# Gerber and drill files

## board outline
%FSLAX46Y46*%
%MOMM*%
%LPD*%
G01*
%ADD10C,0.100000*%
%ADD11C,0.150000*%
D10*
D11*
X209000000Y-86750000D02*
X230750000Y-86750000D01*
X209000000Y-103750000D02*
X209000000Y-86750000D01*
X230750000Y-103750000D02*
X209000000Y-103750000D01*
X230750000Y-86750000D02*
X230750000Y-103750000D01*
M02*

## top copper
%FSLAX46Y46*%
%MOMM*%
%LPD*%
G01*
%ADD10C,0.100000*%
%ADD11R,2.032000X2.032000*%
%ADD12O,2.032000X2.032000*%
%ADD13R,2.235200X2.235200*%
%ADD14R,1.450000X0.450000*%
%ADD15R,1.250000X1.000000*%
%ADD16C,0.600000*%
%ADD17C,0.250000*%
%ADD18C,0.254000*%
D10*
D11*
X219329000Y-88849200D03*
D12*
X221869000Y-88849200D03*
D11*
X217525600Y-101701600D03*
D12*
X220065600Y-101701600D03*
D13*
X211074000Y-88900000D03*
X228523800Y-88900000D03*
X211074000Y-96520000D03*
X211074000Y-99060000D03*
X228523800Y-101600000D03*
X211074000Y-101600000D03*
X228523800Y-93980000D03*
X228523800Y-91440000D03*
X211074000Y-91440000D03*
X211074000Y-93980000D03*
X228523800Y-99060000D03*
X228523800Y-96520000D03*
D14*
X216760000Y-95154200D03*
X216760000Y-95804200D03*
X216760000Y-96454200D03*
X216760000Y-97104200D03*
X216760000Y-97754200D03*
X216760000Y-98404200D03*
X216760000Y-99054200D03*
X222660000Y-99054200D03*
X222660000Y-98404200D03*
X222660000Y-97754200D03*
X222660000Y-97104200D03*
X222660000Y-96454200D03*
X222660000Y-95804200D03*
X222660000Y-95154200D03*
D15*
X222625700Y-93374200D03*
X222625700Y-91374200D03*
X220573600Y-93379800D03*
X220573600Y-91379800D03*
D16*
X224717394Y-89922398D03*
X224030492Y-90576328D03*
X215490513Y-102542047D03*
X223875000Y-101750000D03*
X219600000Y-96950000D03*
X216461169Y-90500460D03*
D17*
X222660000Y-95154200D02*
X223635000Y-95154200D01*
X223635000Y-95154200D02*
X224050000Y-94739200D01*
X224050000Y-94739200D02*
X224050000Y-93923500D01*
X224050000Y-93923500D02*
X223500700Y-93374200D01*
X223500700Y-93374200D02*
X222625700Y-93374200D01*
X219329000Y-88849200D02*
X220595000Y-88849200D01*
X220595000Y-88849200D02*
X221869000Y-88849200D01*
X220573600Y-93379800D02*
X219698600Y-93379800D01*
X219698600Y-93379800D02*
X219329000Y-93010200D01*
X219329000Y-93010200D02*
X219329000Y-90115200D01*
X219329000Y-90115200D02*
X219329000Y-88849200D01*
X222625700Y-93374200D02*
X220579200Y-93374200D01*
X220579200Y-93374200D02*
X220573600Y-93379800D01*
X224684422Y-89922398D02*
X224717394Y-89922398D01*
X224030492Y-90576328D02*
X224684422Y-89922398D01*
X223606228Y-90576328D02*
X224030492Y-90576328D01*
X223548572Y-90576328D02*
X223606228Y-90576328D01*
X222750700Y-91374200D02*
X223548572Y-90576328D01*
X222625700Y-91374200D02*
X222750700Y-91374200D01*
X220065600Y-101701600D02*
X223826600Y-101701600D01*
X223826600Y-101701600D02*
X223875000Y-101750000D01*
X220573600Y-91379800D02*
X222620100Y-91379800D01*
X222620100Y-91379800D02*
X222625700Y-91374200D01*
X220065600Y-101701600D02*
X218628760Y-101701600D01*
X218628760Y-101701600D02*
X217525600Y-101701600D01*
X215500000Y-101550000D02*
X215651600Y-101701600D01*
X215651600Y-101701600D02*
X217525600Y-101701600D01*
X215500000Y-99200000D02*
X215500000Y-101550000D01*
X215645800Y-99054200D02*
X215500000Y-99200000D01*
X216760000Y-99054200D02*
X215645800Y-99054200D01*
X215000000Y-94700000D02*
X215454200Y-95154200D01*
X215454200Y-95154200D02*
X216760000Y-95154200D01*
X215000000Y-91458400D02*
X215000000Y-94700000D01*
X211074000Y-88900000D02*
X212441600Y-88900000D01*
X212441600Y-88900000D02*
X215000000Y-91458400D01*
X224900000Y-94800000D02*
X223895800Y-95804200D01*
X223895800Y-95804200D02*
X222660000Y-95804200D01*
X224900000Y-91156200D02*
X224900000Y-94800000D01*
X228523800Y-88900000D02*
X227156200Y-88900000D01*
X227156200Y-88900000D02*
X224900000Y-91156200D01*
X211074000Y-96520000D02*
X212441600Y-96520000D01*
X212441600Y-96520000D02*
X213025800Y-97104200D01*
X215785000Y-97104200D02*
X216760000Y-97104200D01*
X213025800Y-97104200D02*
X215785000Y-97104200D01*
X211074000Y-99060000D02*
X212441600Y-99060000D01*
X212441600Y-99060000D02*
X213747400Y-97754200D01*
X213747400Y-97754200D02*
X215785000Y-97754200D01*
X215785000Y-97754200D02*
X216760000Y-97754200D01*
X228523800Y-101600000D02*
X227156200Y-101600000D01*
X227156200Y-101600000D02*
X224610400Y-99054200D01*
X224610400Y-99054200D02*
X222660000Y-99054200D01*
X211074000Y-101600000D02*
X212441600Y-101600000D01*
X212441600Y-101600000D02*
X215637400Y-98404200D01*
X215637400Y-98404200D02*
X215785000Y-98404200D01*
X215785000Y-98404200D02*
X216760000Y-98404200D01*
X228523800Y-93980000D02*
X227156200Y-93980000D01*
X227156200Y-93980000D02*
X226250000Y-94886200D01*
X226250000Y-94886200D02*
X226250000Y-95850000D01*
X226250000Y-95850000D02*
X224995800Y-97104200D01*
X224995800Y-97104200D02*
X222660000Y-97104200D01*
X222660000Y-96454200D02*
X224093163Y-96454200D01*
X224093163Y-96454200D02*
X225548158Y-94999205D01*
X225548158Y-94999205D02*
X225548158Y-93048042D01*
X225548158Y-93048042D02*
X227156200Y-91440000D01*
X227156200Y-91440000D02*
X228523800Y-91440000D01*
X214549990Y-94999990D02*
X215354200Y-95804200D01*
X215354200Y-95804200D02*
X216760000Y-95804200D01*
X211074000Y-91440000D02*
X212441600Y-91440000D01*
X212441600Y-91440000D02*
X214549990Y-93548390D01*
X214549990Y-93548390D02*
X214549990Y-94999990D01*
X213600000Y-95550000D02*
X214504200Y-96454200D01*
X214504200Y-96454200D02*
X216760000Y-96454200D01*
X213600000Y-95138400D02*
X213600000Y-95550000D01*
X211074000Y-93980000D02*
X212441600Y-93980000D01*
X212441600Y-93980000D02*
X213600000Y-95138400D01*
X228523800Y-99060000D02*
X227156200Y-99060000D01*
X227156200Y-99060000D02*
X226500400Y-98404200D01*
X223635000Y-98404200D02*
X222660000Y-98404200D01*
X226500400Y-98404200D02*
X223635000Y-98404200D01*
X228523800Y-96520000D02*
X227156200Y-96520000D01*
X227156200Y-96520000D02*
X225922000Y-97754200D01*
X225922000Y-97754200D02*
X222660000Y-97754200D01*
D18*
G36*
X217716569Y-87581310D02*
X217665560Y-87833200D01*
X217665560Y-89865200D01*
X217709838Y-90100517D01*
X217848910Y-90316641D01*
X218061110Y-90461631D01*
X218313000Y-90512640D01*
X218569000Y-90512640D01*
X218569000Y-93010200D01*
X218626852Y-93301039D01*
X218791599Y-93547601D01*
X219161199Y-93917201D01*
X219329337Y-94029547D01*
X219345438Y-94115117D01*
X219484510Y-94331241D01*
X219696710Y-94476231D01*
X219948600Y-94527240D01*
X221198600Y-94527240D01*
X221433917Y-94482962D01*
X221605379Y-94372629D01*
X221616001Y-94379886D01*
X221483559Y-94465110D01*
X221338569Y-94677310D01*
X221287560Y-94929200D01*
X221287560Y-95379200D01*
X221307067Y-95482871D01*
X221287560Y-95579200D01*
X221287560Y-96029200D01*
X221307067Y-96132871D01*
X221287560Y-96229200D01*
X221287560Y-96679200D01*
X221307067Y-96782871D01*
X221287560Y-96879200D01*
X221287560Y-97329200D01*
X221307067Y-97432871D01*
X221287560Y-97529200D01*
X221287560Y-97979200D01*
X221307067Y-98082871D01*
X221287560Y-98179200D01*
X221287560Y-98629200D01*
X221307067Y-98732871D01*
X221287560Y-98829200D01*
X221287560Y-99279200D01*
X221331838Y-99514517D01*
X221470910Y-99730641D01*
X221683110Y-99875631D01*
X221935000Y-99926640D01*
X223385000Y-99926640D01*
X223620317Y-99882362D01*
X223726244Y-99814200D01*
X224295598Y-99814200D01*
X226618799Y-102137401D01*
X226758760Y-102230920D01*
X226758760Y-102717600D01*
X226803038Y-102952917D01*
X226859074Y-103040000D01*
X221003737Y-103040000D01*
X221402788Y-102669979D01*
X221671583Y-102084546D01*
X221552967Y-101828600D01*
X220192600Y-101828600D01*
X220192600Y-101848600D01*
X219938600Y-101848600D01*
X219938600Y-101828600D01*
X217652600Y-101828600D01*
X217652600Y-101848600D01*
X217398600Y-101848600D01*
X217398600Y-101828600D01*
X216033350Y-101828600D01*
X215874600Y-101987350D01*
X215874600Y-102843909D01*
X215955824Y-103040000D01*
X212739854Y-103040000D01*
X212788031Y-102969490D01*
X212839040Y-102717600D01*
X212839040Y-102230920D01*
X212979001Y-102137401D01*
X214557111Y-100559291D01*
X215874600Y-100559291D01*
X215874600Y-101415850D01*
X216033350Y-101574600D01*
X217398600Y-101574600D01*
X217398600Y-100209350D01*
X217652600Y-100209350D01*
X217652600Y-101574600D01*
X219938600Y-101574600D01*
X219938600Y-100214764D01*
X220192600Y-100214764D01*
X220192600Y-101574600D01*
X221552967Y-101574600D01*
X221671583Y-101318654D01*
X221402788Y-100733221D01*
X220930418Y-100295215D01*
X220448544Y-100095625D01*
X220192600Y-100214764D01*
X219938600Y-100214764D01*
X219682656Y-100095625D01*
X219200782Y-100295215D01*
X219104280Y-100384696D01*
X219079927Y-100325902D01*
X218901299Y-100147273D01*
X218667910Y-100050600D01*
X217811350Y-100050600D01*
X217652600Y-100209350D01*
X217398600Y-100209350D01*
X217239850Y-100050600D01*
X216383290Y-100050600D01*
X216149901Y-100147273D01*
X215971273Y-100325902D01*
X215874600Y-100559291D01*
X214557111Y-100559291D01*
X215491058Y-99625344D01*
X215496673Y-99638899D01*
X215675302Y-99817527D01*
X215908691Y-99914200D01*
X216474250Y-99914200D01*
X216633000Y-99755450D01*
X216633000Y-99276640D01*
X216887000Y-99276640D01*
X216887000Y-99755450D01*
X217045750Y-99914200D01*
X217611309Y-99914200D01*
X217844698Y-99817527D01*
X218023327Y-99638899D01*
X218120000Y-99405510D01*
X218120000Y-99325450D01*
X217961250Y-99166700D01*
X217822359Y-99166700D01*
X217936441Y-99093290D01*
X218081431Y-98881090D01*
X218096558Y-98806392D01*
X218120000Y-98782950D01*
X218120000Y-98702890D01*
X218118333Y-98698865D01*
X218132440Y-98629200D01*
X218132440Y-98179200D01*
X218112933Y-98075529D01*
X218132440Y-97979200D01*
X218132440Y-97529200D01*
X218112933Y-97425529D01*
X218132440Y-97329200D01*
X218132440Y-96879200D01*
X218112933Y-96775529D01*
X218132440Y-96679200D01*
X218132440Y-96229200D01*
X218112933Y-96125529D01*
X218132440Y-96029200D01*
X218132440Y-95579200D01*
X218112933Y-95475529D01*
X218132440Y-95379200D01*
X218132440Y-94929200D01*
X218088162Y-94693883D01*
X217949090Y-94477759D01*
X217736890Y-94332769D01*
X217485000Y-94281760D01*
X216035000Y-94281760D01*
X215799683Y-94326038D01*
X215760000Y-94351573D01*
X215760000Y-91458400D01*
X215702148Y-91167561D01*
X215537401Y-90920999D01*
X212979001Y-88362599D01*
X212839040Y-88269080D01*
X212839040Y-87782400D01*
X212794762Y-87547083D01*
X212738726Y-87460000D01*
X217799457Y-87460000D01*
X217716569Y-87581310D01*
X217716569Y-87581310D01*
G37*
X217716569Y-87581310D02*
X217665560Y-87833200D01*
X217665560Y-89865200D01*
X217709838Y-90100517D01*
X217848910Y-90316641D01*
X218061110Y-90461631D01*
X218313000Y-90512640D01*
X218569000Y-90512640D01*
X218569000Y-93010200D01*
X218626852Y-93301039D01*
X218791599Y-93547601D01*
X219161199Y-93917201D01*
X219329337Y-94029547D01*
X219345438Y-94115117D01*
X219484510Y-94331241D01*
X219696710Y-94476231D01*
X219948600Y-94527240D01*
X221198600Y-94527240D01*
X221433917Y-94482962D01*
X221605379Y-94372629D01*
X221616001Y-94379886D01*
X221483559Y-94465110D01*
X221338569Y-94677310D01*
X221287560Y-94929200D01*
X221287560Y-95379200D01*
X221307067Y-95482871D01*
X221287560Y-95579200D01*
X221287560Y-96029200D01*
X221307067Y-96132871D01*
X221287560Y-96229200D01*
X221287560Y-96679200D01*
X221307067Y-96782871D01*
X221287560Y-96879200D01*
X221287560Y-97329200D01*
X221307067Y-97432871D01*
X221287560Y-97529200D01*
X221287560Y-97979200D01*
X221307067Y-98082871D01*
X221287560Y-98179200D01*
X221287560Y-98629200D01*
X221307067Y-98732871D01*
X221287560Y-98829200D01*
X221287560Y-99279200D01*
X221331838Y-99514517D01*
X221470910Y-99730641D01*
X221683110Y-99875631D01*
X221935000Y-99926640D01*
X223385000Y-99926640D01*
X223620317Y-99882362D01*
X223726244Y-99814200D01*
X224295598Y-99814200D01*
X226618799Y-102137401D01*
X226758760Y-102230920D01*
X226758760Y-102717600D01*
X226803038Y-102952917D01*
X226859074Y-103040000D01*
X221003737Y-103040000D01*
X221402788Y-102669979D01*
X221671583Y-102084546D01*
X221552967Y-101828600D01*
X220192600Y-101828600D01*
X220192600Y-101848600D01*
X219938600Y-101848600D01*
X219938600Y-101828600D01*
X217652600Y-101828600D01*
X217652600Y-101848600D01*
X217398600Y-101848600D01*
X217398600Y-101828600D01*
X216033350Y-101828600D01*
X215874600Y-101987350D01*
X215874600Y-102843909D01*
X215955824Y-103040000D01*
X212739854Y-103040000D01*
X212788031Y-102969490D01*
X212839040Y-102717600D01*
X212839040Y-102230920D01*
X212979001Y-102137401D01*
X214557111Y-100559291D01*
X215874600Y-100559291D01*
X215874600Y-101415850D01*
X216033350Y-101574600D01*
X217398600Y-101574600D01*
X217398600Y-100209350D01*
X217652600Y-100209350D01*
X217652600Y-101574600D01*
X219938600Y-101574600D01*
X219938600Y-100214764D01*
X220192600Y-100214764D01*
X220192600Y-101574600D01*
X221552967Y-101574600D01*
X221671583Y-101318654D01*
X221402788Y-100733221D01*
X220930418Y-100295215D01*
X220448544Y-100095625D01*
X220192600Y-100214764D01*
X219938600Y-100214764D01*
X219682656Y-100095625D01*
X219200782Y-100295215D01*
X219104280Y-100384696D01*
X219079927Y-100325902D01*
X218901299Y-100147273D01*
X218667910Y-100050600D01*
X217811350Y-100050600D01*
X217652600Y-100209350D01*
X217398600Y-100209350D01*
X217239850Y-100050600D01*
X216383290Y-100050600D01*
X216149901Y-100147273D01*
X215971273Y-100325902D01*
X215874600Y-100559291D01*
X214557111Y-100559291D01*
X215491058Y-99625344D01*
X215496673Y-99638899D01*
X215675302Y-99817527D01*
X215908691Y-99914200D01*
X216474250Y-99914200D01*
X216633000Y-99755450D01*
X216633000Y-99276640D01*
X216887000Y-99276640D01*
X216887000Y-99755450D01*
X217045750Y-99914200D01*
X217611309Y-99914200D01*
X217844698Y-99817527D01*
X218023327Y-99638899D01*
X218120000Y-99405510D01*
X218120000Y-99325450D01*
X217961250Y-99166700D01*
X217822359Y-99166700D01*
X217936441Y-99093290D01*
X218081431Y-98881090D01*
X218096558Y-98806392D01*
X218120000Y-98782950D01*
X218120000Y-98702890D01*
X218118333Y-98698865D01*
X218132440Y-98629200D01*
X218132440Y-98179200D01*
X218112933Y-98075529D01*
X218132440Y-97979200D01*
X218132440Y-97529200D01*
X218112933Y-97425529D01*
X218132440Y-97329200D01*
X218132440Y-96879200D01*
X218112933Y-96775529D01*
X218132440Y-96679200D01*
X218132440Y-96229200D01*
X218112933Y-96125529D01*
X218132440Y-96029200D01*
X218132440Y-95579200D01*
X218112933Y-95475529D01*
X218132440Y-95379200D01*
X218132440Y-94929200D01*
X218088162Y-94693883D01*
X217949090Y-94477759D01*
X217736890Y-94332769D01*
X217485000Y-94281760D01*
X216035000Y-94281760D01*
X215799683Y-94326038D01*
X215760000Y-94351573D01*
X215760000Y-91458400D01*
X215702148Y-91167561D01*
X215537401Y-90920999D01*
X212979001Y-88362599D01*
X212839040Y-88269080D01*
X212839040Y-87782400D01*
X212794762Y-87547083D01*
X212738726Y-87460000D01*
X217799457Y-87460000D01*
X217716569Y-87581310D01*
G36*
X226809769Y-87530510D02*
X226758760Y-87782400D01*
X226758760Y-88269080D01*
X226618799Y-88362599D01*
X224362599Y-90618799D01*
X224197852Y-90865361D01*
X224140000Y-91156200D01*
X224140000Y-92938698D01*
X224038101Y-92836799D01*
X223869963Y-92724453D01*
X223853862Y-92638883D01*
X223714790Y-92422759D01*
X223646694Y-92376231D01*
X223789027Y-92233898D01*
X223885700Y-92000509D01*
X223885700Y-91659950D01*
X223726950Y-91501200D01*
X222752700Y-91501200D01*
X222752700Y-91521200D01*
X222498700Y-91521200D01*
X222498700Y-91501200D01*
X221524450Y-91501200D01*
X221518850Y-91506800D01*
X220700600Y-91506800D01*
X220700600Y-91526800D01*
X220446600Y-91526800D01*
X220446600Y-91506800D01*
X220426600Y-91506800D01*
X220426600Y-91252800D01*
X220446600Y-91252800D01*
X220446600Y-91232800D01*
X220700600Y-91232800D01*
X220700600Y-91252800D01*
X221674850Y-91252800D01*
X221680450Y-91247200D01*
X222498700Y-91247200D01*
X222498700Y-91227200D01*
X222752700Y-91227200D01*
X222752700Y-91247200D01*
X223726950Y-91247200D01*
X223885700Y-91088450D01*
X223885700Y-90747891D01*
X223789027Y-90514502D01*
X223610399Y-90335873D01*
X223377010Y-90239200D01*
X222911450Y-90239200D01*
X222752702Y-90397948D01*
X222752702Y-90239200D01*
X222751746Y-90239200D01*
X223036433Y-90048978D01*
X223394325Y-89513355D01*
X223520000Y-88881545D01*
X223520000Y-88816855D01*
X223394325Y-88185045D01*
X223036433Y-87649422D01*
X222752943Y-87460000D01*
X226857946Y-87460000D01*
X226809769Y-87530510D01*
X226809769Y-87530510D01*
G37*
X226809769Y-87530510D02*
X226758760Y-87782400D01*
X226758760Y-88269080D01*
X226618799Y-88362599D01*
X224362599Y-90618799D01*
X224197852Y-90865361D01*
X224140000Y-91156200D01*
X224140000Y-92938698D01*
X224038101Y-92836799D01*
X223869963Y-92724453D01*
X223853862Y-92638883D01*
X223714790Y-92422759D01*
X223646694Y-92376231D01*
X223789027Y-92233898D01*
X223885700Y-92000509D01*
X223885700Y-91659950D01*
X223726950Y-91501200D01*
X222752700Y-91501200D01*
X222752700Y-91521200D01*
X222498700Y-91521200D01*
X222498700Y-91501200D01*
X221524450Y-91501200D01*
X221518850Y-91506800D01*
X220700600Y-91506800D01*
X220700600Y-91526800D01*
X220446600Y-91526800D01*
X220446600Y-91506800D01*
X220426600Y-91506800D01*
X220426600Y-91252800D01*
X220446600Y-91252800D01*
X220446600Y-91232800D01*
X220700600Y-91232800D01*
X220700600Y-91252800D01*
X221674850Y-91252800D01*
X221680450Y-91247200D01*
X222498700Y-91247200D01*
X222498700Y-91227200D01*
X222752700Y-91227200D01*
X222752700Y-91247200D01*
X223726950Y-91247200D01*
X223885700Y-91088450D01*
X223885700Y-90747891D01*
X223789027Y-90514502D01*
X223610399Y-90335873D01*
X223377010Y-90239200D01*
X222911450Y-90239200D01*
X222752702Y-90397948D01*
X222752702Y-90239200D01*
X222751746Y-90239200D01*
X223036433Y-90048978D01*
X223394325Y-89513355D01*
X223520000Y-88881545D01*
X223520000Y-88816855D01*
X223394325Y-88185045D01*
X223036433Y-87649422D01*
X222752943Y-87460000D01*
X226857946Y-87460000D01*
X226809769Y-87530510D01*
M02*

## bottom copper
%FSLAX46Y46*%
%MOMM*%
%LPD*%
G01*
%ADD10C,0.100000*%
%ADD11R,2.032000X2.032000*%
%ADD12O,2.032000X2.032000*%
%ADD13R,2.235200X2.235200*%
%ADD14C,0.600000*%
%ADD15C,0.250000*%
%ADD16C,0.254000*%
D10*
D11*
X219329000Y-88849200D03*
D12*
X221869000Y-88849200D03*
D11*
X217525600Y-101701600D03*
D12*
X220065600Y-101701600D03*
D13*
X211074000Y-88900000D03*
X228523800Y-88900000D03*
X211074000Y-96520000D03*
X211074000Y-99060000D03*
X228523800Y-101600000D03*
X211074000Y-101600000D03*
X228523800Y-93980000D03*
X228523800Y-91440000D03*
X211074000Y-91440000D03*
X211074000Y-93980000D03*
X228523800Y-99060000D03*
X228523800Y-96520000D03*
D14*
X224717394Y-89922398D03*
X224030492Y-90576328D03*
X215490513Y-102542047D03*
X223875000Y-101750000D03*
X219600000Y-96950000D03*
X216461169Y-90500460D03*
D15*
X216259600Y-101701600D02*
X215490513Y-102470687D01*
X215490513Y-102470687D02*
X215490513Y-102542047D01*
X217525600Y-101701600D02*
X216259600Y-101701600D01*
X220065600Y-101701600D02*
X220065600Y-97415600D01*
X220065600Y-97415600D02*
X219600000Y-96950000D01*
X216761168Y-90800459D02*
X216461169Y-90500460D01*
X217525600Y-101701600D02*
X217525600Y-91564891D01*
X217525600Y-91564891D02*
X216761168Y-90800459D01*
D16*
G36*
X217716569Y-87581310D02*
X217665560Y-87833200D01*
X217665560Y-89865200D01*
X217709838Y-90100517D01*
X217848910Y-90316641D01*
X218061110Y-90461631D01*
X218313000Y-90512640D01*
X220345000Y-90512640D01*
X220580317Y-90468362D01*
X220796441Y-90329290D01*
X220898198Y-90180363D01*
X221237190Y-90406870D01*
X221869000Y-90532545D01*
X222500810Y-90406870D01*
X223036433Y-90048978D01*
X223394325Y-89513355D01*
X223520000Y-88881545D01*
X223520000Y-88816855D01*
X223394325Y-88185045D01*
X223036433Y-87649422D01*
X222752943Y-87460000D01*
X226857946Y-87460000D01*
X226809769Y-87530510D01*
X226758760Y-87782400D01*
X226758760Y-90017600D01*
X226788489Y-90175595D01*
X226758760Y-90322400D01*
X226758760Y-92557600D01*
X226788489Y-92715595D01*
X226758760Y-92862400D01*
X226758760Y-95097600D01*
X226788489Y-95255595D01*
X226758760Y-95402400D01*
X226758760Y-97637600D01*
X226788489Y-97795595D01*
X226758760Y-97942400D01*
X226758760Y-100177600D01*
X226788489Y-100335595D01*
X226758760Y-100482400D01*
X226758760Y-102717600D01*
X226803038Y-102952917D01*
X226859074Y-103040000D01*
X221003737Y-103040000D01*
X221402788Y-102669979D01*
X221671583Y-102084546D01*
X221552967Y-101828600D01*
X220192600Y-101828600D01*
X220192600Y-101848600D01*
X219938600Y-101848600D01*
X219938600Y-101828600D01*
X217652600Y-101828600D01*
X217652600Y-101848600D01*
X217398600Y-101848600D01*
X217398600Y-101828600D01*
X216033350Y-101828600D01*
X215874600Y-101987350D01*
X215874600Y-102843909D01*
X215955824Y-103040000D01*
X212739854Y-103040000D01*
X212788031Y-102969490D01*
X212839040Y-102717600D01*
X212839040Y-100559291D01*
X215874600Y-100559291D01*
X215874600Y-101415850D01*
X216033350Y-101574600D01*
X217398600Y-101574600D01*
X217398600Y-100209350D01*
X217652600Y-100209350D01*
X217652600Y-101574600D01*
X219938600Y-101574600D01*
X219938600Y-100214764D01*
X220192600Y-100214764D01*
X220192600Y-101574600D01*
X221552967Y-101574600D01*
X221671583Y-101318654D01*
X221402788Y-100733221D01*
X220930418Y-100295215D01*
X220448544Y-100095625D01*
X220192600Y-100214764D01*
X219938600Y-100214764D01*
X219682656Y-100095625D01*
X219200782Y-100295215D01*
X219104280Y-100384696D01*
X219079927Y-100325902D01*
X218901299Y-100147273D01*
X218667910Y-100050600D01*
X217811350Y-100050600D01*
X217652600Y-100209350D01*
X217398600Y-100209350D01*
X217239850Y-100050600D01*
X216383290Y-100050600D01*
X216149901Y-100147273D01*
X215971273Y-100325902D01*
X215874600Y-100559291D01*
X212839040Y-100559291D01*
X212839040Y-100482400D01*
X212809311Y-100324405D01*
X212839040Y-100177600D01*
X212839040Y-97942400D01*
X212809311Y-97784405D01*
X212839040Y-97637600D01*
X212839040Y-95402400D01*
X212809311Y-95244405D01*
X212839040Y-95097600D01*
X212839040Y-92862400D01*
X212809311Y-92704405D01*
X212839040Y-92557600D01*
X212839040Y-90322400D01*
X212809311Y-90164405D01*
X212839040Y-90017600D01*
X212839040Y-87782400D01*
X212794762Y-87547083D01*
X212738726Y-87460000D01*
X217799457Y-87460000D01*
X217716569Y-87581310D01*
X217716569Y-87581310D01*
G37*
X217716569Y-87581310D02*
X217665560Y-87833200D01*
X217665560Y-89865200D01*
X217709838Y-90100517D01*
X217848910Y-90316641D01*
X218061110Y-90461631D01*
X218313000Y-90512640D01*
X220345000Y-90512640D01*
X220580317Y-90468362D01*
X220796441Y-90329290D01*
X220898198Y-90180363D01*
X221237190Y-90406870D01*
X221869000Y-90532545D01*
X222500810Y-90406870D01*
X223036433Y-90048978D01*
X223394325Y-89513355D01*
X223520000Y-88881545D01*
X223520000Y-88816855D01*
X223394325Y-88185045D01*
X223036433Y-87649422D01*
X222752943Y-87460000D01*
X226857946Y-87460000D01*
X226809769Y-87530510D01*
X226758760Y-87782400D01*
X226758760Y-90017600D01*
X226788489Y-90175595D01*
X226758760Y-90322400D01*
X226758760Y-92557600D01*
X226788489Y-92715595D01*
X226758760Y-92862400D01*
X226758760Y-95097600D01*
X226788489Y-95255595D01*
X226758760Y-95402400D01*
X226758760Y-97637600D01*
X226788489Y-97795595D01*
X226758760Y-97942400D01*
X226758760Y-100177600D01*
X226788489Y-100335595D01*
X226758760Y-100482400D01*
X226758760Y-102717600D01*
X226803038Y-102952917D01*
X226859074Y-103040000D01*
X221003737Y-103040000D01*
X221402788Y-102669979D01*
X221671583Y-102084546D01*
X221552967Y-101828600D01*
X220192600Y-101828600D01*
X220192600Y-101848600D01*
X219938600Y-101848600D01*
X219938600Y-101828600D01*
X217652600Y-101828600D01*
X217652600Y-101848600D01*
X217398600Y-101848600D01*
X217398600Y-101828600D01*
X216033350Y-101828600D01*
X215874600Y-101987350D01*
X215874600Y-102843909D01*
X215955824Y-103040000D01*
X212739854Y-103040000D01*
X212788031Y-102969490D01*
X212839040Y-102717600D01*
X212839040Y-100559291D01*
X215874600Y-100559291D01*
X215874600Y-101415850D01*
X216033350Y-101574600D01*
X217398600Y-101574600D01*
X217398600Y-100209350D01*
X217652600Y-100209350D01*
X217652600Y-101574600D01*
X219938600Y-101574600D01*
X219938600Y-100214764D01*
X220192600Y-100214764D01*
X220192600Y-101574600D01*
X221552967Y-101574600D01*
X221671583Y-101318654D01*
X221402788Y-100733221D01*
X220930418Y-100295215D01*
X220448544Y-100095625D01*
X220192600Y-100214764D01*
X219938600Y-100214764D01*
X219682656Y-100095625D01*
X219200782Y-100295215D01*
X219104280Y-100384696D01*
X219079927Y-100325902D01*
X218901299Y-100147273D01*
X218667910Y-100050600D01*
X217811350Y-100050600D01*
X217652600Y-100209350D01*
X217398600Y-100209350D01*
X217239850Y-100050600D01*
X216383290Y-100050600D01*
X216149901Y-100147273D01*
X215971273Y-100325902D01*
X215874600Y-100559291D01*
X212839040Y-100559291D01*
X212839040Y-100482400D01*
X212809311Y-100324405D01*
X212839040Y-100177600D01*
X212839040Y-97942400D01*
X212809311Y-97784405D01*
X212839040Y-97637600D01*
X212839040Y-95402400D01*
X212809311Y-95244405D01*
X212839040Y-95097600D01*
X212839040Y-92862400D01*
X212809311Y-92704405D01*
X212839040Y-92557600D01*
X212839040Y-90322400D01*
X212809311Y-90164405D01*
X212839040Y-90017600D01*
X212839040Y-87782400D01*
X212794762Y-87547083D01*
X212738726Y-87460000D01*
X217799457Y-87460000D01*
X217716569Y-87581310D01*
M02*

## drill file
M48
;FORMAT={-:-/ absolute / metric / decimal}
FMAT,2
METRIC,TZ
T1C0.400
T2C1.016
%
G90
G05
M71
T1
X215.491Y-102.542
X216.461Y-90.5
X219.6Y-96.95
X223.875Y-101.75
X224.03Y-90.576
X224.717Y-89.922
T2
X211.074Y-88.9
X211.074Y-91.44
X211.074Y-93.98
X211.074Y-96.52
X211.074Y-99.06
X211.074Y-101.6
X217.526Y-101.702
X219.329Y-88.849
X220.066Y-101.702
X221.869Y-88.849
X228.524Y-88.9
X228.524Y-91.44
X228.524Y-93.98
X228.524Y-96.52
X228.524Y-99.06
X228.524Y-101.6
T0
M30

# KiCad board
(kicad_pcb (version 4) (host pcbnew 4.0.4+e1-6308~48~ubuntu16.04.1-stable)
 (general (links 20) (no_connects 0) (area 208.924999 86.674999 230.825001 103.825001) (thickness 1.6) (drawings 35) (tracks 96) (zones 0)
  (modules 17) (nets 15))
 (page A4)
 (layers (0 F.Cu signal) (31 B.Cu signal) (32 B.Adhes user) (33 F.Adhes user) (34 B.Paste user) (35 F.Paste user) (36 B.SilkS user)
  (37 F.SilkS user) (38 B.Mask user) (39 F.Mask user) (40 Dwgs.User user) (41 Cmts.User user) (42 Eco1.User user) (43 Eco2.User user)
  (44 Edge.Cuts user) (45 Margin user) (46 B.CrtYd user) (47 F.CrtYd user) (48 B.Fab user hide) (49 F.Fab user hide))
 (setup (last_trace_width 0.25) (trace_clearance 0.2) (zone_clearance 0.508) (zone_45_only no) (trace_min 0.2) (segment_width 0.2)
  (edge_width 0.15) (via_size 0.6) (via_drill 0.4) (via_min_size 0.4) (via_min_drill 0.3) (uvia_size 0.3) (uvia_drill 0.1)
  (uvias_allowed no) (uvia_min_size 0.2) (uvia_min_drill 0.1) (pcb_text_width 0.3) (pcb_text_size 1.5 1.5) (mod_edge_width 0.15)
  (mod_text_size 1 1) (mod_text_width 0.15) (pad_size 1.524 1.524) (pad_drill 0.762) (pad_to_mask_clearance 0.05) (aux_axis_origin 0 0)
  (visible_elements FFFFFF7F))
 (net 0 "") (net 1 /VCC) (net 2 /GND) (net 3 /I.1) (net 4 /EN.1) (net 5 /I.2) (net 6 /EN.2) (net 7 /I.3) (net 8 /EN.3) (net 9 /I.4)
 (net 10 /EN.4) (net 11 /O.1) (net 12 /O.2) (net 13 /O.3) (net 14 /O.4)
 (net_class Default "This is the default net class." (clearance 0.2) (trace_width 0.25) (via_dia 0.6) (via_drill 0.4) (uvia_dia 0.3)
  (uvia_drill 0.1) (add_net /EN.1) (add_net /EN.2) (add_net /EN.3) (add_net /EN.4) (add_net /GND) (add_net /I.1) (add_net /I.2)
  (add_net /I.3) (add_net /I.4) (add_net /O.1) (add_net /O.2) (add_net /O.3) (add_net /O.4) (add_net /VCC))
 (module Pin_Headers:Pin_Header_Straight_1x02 (layer F.Cu) (at 219.329 88.8492 90)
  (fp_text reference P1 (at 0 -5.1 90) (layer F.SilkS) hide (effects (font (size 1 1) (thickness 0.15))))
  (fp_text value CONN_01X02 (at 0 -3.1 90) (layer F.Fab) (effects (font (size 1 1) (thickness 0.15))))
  (pad 1 thru_hole rect (at 0 0 90) (size 2.032 2.032) (drill 1.016) (layers *.Cu *.Mask F.SilkS) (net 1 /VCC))
  (pad 2 thru_hole oval (at 0 2.54 90) (size 2.032 2.032) (drill 1.016) (layers *.Cu *.Mask F.SilkS) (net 1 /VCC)))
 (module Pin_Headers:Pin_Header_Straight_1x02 (layer F.Cu) (at 217.5256 101.7016 90)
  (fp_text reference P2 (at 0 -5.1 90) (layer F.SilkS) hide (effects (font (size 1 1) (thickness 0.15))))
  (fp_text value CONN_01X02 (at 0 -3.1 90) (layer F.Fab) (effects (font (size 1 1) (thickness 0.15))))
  (pad 1 thru_hole rect (at 0 0 90) (size 2.032 2.032) (drill 1.016) (layers *.Cu *.Mask F.SilkS) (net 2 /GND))
  (pad 2 thru_hole oval (at 0 2.54 90) (size 2.032 2.032) (drill 1.016) (layers *.Cu *.Mask F.SilkS) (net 2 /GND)))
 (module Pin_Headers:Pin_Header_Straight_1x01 (layer F.Cu) (at 211.074 88.9 90)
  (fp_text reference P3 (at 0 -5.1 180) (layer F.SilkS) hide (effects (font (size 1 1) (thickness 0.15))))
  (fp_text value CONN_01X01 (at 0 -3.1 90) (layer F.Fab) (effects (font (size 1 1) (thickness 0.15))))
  (pad 1 thru_hole rect (at 0 0 90) (size 2.2352 2.2352) (drill 1.016) (layers *.Cu *.Mask F.SilkS) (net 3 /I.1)))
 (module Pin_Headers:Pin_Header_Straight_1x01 (layer F.Cu) (at 228.5238 88.9)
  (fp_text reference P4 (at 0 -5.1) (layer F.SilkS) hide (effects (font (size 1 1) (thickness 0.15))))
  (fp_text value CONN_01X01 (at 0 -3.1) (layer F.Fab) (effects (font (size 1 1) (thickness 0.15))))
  (pad 1 thru_hole rect (at 0 0) (size 2.2352 2.2352) (drill 1.016) (layers *.Cu *.Mask F.SilkS) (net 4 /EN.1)))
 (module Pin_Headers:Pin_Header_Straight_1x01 (layer F.Cu) (at 211.074 96.52 270)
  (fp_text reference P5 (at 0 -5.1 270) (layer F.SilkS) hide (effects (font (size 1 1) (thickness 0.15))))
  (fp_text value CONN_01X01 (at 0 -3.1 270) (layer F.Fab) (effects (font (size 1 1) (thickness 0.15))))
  (pad 1 thru_hole rect (at 0 0 270) (size 2.2352 2.2352) (drill 1.016) (layers *.Cu *.Mask F.SilkS) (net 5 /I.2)))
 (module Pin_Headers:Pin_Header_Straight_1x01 (layer F.Cu) (at 211.074 99.06 90)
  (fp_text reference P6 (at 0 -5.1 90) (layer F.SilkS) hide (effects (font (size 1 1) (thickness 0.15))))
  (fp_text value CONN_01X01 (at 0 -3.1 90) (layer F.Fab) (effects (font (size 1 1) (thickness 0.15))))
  (pad 1 thru_hole rect (at 0 0 90) (size 2.2352 2.2352) (drill 1.016) (layers *.Cu *.Mask F.SilkS) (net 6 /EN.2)))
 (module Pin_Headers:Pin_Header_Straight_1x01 (layer F.Cu) (at 228.5238 101.6 180)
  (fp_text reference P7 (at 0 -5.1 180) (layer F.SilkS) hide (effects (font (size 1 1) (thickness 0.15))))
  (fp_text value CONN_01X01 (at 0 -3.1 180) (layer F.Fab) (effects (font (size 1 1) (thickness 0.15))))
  (pad 1 thru_hole rect (at 0 0 180) (size 2.2352 2.2352) (drill 1.016) (layers *.Cu *.Mask F.SilkS) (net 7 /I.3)))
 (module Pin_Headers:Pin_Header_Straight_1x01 (layer F.Cu) (at 211.074 101.6 270)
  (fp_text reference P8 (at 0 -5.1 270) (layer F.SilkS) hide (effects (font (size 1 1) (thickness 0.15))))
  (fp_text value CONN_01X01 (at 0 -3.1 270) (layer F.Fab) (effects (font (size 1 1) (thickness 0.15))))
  (pad 1 thru_hole rect (at 0 0 270) (size 2.2352 2.2352) (drill 1.016) (layers *.Cu *.Mask F.SilkS) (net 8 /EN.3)))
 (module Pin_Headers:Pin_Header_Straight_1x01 (layer F.Cu) (at 228.5238 93.98)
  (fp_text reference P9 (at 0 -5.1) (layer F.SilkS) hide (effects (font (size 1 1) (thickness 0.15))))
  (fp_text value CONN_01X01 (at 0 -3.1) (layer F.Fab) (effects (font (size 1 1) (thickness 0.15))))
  (pad 1 thru_hole rect (at 0 0) (size 2.2352 2.2352) (drill 1.016) (layers *.Cu *.Mask F.SilkS) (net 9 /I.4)))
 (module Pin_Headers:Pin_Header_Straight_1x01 (layer F.Cu) (at 228.5238 91.44 180)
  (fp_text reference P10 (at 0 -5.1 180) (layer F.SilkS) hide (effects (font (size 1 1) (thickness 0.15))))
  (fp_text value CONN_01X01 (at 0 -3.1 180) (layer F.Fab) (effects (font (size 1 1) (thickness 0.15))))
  (pad 1 thru_hole rect (at 0 0 180) (size 2.2352 2.2352) (drill 1.016) (layers *.Cu *.Mask F.SilkS) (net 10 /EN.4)))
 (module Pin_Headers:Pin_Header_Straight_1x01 (layer F.Cu) (at 211.074 91.44 270)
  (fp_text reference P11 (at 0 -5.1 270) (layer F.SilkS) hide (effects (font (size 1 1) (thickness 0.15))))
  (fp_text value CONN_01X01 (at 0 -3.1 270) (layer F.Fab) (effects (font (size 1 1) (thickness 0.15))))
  (pad 1 thru_hole rect (at 0 0 270) (size 2.2352 2.2352) (drill 1.016) (layers *.Cu *.Mask F.SilkS) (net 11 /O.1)))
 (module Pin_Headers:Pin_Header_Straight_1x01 (layer F.Cu) (at 211.074 93.98 90)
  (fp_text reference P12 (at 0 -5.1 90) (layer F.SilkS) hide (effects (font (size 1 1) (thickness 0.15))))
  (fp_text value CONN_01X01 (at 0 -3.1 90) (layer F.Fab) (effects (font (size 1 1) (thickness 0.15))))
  (pad 1 thru_hole rect (at 0 0 90) (size 2.2352 2.2352) (drill 1.016) (layers *.Cu *.Mask F.SilkS) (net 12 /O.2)))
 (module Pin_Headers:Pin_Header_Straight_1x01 (layer F.Cu) (at 228.5238 99.06)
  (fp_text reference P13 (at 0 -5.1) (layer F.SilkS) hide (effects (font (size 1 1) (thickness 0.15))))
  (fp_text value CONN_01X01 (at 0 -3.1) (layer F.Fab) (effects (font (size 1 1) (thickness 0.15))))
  (pad 1 thru_hole rect (at 0 0) (size 2.2352 2.2352) (drill 1.016) (layers *.Cu *.Mask F.SilkS) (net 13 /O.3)))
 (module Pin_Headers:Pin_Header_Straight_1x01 (layer F.Cu) (at 228.5238 96.52 180)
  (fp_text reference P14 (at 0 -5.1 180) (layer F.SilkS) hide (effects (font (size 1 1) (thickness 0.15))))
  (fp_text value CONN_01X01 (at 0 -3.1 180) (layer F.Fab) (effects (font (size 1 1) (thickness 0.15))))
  (pad 1 thru_hole rect (at 0 0 180) (size 2.2352 2.2352) (drill 1.016) (layers *.Cu *.Mask F.SilkS) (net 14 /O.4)))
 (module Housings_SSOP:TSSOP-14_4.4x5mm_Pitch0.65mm (layer F.Cu) (at 219.71 97.1042)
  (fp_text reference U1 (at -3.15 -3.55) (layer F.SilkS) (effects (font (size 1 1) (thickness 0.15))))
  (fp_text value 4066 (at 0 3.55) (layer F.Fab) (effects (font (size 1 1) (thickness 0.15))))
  (pad 1 smd rect (at -2.95 -1.95) (size 1.45 0.45) (layers F.Cu F.Paste F.Mask) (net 3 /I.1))
  (pad 2 smd rect (at -2.95 -1.3) (size 1.45 0.45) (layers F.Cu F.Paste F.Mask) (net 11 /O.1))
  (pad 3 smd rect (at -2.95 -0.65) (size 1.45 0.45) (layers F.Cu F.Paste F.Mask) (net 12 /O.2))
  (pad 4 smd rect (at -2.95 0) (size 1.45 0.45) (layers F.Cu F.Paste F.Mask) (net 5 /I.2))
  (pad 5 smd rect (at -2.95 0.65) (size 1.45 0.45) (layers F.Cu F.Paste F.Mask) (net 6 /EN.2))
  (pad 6 smd rect (at -2.95 1.3) (size 1.45 0.45) (layers F.Cu F.Paste F.Mask) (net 8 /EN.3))
  (pad 7 smd rect (at -2.95 1.95) (size 1.45 0.45) (layers F.Cu F.Paste F.Mask) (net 2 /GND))
  (pad 8 smd rect (at 2.95 1.95) (size 1.45 0.45) (layers F.Cu F.Paste F.Mask) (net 7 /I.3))
  (pad 9 smd rect (at 2.95 1.3) (size 1.45 0.45) (layers F.Cu F.Paste F.Mask) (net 13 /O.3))
  (pad 10 smd rect (at 2.95 0.65) (size 1.45 0.45) (layers F.Cu F.Paste F.Mask) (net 14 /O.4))
  (pad 11 smd rect (at 2.95 0) (size 1.45 0.45) (layers F.Cu F.Paste F.Mask) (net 9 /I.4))
  (pad 12 smd rect (at 2.95 -0.65) (size 1.45 0.45) (layers F.Cu F.Paste F.Mask) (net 10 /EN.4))
  (pad 13 smd rect (at 2.95 -1.3) (size 1.45 0.45) (layers F.Cu F.Paste F.Mask) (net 4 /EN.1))
  (pad 14 smd rect (at 2.95 -1.95) (size 1.45 0.45) (layers F.Cu F.Paste F.Mask) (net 1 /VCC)))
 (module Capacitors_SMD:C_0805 (layer F.Cu) (at 222.6257 92.3742 90)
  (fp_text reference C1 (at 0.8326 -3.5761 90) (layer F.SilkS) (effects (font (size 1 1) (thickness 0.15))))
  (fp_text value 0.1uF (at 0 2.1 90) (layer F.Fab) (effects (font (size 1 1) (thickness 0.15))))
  (pad 1 smd rect (at -1 0 90) (size 1 1.25) (layers F.Cu F.Paste F.Mask) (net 1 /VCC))
  (pad 2 smd rect (at 1 0 90) (size 1 1.25) (layers F.Cu F.Paste F.Mask) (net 2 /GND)))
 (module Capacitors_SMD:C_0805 (layer F.Cu) (at 220.5736 92.3798 90)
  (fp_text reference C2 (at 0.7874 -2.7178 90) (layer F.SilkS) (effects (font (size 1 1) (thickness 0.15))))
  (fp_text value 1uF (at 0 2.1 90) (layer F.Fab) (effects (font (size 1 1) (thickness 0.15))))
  (pad 1 smd rect (at -1 0 90) (size 1 1.25) (layers F.Cu F.Paste F.Mask) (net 1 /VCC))
  (pad 2 smd rect (at 1 0 90) (size 1 1.25) (layers F.Cu F.Paste F.Mask) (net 2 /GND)))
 (gr_line (start 209 86.75) (end 230.75 86.75) (layer Edge.Cuts) (width 0.15))
 (gr_line (start 209 103.75) (end 209 86.75) (layer Edge.Cuts) (width 0.15))
 (gr_line (start 230.75 103.75) (end 209 103.75) (layer Edge.Cuts) (width 0.15))
 (gr_line (start 230.75 86.75) (end 230.75 103.75) (layer Edge.Cuts) (width 0.15))
 (segment (start 222.66 95.1542) (end 223.635 95.1542) (width 0.25) (layer F.Cu) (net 1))
 (segment (start 223.635 95.1542) (end 224.05 94.7392) (width 0.25) (layer F.Cu) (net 1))
 (segment (start 224.05 94.7392) (end 224.05 93.9235) (width 0.25) (layer F.Cu) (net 1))
 (segment (start 224.05 93.9235) (end 223.5007 93.3742) (width 0.25) (layer F.Cu) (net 1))
 (segment (start 223.5007 93.3742) (end 222.6257 93.3742) (width 0.25) (layer F.Cu) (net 1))
 (segment (start 219.329 88.8492) (end 220.595 88.8492) (width 0.25) (layer F.Cu) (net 1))
 (segment (start 220.595 88.8492) (end 221.869 88.8492) (width 0.25) (layer F.Cu) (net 1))
 (segment (start 220.5736 93.3798) (end 219.6986 93.3798) (width 0.25) (layer F.Cu) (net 1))
 (segment (start 219.6986 93.3798) (end 219.329 93.0102) (width 0.25) (layer F.Cu) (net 1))
 (segment (start 219.329 93.0102) (end 219.329 90.1152) (width 0.25) (layer F.Cu) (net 1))
 (segment (start 219.329 90.1152) (end 219.329 88.8492) (width 0.25) (layer F.Cu) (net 1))
 (segment (start 222.6257 93.3742) (end 220.5792 93.3742) (width 0.25) (layer F.Cu) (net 1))
 (segment (start 220.5792 93.3742) (end 220.5736 93.3798) (width 0.25) (layer F.Cu) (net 1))
 (segment (start 224.684422 89.922398) (end 224.717394 89.922398) (width 0.25) (layer F.Cu) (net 2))
 (segment (start 224.030492 90.576328) (end 224.684422 89.922398) (width 0.25) (layer F.Cu) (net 2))
 (via (at 224.717394 89.922398) (size 0.6) (drill 0.4) (layers F.Cu B.Cu) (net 2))
 (segment (start 223.606228 90.576328) (end 224.030492 90.576328) (width 0.25) (layer F.Cu) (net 2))
 (segment (start 223.548572 90.576328) (end 223.606228 90.576328) (width 0.25) (layer F.Cu) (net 2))
 (segment (start 222.7507 91.3742) (end 223.548572 90.576328) (width 0.25) (layer F.Cu) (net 2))
 (segment (start 222.6257 91.3742) (end 222.7507 91.3742) (width 0.25) (layer F.Cu) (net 2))
 (via (at 224.030492 90.576328) (size 0.6) (drill 0.4) (layers F.Cu B.Cu) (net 2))
 (segment (start 216.2596 101.7016) (end 215.490513 102.470687) (width 0.25) (layer B.Cu) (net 2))
 (segment (start 215.490513 102.470687) (end 215.490513 102.542047) (width 0.25) (layer B.Cu) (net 2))
 (segment (start 217.5256 101.7016) (end 216.2596 101.7016) (width 0.25) (layer B.Cu) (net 2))
 (via (at 215.490513 102.542047) (size 0.6) (drill 0.4) (layers F.Cu B.Cu) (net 2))
 (segment (start 220.0656 101.7016) (end 223.8266 101.7016) (width 0.25) (layer F.Cu) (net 2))
 (segment (start 223.8266 101.7016) (end 223.875 101.75) (width 0.25) (layer F.Cu) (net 2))
 (via (at 223.875 101.75) (size 0.6) (drill 0.4) (layers F.Cu B.Cu) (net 2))
 (segment (start 220.0656 101.7016) (end 220.0656 97.4156) (width 0.25) (layer B.Cu) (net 2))
 (segment (start 220.0656 97.4156) (end 219.6 96.95) (width 0.25) (layer B.Cu) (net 2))
 (via (at 219.6 96.95) (size 0.6) (drill 0.4) (layers F.Cu B.Cu) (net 2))
 (segment (start 216.761168 90.800459) (end 216.461169 90.50046) (width 0.25) (layer B.Cu) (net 2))
 (segment (start 217.5256 101.7016) (end 217.5256 91.564891) (width 0.25) (layer B.Cu) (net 2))
 (segment (start 217.5256 91.564891) (end 216.761168 90.800459) (width 0.25) (layer B.Cu) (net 2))
 (via (at 216.461169 90.50046) (size 0.6) (drill 0.4) (layers F.Cu B.Cu) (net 2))
 (segment (start 220.5736 91.3798) (end 222.6201 91.3798) (width 0.25) (layer F.Cu) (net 2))
 (segment (start 222.6201 91.3798) (end 222.6257 91.3742) (width 0.25) (layer F.Cu) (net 2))
 (segment (start 220.0656 101.7016) (end 218.62876 101.7016) (width 0.25) (layer F.Cu) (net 2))
 (segment (start 218.62876 101.7016) (end 217.5256 101.7016) (width 0.25) (layer F.Cu) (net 2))
 (segment (start 215.5 101.55) (end 215.6516 101.7016) (width 0.25) (layer F.Cu) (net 2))
 (segment (start 215.6516 101.7016) (end 217.5256 101.7016) (width 0.25) (layer F.Cu) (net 2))
 (segment (start 215.5 99.2) (end 215.5 101.55) (width 0.25) (layer F.Cu) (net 2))
 (segment (start 215.6458 99.0542) (end 215.5 99.2) (width 0.25) (layer F.Cu) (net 2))
 (segment (start 216.76 99.0542) (end 215.6458 99.0542) (width 0.25) (layer F.Cu) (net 2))
 (segment (start 215 94.7) (end 215.4542 95.1542) (width 0.25) (layer F.Cu) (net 3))
 (segment (start 215.4542 95.1542) (end 216.76 95.1542) (width 0.25) (layer F.Cu) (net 3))
 (segment (start 215 91.4584) (end 215 94.7) (width 0.25) (layer F.Cu) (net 3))
 (segment (start 211.074 88.9) (end 212.4416 88.9) (width 0.25) (layer F.Cu) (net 3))
 (segment (start 212.4416 88.9) (end 215 91.4584) (width 0.25) (layer F.Cu) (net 3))
 (segment (start 224.9 94.8) (end 223.8958 95.8042) (width 0.25) (layer F.Cu) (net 4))
 (segment (start 223.8958 95.8042) (end 222.66 95.8042) (width 0.25) (layer F.Cu) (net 4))
 (segment (start 224.9 91.1562) (end 224.9 94.8) (width 0.25) (layer F.Cu) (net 4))
 (segment (start 228.5238 88.9) (end 227.1562 88.9) (width 0.25) (layer F.Cu) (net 4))
 (segment (start 227.1562 88.9) (end 224.9 91.1562) (width 0.25) (layer F.Cu) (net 4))
 (segment (start 211.074 96.52) (end 212.4416 96.52) (width 0.25) (layer F.Cu) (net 5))
 (segment (start 212.4416 96.52) (end 213.0258 97.1042) (width 0.25) (layer F.Cu) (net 5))
 (segment (start 215.785 97.1042) (end 216.76 97.1042) (width 0.25) (layer F.Cu) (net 5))
 (segment (start 213.0258 97.1042) (end 215.785 97.1042) (width 0.25) (layer F.Cu) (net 5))
 (segment (start 211.074 99.06) (end 212.4416 99.06) (width 0.25) (layer F.Cu) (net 6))
 (segment (start 212.4416 99.06) (end 213.7474 97.7542) (width 0.25) (layer F.Cu) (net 6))
 (segment (start 213.7474 97.7542) (end 215.785 97.7542) (width 0.25) (layer F.Cu) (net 6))
 (segment (start 215.785 97.7542) (end 216.76 97.7542) (width 0.25) (layer F.Cu) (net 6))
 (segment (start 228.5238 101.6) (end 227.1562 101.6) (width 0.25) (layer F.Cu) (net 7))
 (segment (start 227.1562 101.6) (end 224.6104 99.0542) (width 0.25) (layer F.Cu) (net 7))
 (segment (start 224.6104 99.0542) (end 222.66 99.0542) (width 0.25) (layer F.Cu) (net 7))
 (segment (start 211.074 101.6) (end 212.4416 101.6) (width 0.25) (layer F.Cu) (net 8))
 (segment (start 212.4416 101.6) (end 215.6374 98.4042) (width 0.25) (layer F.Cu) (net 8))
 (segment (start 215.6374 98.4042) (end 215.785 98.4042) (width 0.25) (layer F.Cu) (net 8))
 (segment (start 215.785 98.4042) (end 216.76 98.4042) (width 0.25) (layer F.Cu) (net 8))
 (segment (start 228.5238 93.98) (end 227.1562 93.98) (width 0.25) (layer F.Cu) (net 9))
 (segment (start 227.1562 93.98) (end 226.25 94.8862) (width 0.25) (layer F.Cu) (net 9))
 (segment (start 226.25 94.8862) (end 226.25 95.85) (width 0.25) (layer F.Cu) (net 9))
 (segment (start 226.25 95.85) (end 224.9958 97.1042) (width 0.25) (layer F.Cu) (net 9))
 (segment (start 224.9958 97.1042) (end 222.66 97.1042) (width 0.25) (layer F.Cu) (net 9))
 (segment (start 222.66 96.4542) (end 224.093163 96.4542) (width 0.25) (layer F.Cu) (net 10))
 (segment (start 224.093163 96.4542) (end 225.548158 94.999205) (width 0.25) (layer F.Cu) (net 10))
 (segment (start 225.548158 94.999205) (end 225.548158 93.048042) (width 0.25) (layer F.Cu) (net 10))
 (segment (start 225.548158 93.048042) (end 227.1562 91.44) (width 0.25) (layer F.Cu) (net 10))
 (segment (start 227.1562 91.44) (end 228.5238 91.44) (width 0.25) (layer F.Cu) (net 10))
 (segment (start 214.54999 94.99999) (end 215.3542 95.8042) (width 0.25) (layer F.Cu) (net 11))
 (segment (start 215.3542 95.8042) (end 216.76 95.8042) (width 0.25) (layer F.Cu) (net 11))
 (segment (start 211.074 91.44) (end 212.4416 91.44) (width 0.25) (layer F.Cu) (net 11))
 (segment (start 212.4416 91.44) (end 214.54999 93.54839) (width 0.25) (layer F.Cu) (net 11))
 (segment (start 214.54999 93.54839) (end 214.54999 94.99999) (width 0.25) (layer F.Cu) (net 11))
 (segment (start 213.6 95.55) (end 214.5042 96.4542) (width 0.25) (layer F.Cu) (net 12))
 (segment (start 214.5042 96.4542) (end 216.76 96.4542) (width 0.25) (layer F.Cu) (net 12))
 (segment (start 213.6 95.1384) (end 213.6 95.55) (width 0.25) (layer F.Cu) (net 12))
 (segment (start 211.074 93.98) (end 212.4416 93.98) (width 0.25) (layer F.Cu) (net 12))
 (segment (start 212.4416 93.98) (end 213.6 95.1384) (width 0.25) (layer F.Cu) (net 12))
 (segment (start 228.5238 99.06) (end 227.1562 99.06) (width 0.25) (layer F.Cu) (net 13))
 (segment (start 227.1562 99.06) (end 226.5004 98.4042) (width 0.25) (layer F.Cu) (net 13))
 (segment (start 223.635 98.4042) (end 222.66 98.4042) (width 0.25) (layer F.Cu) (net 13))
 (segment (start 226.5004 98.4042) (end 223.635 98.4042) (width 0.25) (layer F.Cu) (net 13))
 (segment (start 228.5238 96.52) (end 227.1562 96.52) (width 0.25) (layer F.Cu) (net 14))
 (segment (start 227.1562 96.52) (end 225.922 97.7542) (width 0.25) (layer F.Cu) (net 14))
 (segment (start 225.922 97.7542) (end 222.66 97.7542) (width 0.25) (layer F.Cu) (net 14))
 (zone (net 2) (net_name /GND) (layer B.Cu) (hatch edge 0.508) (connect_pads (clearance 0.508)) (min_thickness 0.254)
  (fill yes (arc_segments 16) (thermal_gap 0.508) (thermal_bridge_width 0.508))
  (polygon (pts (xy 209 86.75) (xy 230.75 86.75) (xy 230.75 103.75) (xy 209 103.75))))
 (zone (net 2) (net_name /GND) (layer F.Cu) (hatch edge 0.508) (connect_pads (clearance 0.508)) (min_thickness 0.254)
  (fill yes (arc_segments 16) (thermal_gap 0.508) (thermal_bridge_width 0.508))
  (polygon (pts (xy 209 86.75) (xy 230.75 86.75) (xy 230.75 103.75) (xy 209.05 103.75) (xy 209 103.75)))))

